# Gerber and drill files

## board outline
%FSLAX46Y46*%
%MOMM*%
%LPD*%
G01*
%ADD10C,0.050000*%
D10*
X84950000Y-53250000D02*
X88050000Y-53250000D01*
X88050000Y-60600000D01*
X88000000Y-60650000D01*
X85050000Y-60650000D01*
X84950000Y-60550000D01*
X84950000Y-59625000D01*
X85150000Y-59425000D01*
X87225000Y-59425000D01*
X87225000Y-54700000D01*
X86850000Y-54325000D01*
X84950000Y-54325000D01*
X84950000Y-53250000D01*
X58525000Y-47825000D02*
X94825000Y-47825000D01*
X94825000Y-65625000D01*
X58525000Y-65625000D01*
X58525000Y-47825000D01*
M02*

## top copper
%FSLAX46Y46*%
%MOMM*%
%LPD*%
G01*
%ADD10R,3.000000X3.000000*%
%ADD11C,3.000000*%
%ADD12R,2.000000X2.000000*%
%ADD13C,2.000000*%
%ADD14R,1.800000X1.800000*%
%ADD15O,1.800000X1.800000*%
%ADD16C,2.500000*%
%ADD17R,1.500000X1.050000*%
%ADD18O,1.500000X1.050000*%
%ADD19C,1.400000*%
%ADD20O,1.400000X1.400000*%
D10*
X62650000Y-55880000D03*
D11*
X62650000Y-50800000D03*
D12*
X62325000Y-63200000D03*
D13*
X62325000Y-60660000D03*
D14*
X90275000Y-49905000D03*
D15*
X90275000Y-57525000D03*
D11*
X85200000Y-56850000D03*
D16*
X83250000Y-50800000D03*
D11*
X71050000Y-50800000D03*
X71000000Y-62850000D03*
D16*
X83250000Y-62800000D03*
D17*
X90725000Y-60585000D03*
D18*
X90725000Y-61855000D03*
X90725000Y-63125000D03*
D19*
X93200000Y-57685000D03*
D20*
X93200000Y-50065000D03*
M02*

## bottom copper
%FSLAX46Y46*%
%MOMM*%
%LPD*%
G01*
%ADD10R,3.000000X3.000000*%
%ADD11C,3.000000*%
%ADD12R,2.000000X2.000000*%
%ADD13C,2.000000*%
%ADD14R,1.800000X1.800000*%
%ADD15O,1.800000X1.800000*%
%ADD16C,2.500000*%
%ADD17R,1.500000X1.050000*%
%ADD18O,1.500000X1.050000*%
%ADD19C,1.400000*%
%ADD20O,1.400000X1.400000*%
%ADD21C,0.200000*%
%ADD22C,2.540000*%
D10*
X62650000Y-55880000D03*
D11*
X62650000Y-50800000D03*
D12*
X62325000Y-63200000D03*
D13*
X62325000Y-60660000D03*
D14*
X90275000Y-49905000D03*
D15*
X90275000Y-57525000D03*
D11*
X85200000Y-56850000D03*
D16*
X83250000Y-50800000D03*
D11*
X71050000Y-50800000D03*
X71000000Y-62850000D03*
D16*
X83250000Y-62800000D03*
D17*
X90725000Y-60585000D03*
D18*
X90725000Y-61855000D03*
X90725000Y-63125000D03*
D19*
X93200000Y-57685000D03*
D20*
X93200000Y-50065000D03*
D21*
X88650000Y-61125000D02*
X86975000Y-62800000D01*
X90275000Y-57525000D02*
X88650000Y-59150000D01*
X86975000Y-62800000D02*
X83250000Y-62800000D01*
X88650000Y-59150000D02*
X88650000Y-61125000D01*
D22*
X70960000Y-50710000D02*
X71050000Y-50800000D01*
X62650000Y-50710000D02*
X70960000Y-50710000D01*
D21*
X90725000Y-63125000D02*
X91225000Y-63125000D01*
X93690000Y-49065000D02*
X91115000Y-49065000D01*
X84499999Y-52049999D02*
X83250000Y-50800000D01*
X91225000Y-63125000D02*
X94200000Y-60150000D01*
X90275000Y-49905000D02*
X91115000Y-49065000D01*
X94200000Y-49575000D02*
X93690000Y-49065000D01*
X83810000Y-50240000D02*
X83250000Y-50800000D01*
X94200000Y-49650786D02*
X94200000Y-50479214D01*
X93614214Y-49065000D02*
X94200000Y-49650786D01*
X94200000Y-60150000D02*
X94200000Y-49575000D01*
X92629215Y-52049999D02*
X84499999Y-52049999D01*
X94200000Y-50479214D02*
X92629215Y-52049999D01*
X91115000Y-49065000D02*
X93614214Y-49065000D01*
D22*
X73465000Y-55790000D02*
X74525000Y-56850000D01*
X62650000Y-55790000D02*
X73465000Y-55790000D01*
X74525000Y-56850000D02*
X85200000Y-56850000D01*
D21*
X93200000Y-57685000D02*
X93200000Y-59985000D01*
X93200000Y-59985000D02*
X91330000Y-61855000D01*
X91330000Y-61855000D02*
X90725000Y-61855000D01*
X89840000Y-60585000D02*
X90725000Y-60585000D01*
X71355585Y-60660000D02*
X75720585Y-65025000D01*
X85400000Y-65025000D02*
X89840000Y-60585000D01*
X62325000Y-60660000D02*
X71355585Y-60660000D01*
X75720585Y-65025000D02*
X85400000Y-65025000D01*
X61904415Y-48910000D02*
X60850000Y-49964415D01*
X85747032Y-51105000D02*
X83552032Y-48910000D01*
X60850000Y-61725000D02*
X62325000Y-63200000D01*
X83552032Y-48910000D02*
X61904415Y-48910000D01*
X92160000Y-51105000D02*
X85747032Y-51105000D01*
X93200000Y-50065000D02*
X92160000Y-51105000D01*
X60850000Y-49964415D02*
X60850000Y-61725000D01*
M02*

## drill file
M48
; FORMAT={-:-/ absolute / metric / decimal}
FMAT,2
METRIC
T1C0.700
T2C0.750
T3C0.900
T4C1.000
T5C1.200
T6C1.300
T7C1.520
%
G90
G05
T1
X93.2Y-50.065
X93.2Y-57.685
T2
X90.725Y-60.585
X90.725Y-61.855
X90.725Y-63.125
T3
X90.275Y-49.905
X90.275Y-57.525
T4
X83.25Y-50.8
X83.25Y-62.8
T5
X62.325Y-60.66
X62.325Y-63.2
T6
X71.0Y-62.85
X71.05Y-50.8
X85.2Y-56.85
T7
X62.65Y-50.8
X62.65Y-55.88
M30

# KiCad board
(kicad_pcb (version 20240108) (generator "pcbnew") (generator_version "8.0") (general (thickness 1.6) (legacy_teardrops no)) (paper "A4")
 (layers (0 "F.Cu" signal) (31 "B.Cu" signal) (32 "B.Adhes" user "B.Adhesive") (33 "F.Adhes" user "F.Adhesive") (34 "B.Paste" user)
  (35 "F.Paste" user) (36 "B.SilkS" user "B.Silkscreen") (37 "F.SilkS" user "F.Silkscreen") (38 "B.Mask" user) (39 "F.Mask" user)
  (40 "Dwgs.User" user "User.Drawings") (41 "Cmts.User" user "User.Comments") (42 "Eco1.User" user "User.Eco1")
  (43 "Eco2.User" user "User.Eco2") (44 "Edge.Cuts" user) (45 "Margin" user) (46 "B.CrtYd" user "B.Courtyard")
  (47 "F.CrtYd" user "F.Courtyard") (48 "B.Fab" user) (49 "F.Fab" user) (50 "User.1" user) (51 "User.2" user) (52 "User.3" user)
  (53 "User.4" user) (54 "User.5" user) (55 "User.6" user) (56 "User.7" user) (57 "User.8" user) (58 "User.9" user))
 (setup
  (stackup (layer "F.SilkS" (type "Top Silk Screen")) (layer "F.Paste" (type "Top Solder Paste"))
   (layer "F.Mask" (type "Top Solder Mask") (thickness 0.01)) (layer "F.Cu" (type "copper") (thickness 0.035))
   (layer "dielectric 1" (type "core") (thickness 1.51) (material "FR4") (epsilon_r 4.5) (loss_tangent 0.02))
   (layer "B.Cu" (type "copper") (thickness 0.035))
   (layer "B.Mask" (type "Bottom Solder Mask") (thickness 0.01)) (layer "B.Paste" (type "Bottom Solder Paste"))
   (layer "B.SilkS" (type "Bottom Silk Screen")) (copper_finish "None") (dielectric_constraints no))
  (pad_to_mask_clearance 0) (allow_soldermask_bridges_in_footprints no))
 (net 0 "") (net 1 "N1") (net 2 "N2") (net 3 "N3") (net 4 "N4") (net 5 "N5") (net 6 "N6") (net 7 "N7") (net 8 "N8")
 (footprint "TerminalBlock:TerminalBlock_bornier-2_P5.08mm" (layer "F.Cu") (at 62.65 55.88 90)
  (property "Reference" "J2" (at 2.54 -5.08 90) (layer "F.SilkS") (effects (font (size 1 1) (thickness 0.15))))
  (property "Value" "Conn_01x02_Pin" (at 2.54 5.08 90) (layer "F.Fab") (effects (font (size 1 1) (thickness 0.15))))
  (pad "1" thru_hole rect (at 0 0 90) (size 3 3) (drill 1.52) (layers "*.Cu" "*.Mask") (remove_unused_layers no) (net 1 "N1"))
  (pad "2" thru_hole circle (at 5.08 0 90) (size 3 3) (drill 1.52) (layers "*.Cu" "*.Mask") (remove_unused_layers no) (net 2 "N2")))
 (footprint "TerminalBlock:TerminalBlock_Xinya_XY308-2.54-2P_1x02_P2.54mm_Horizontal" (layer "F.Cu") (at 62.325 63.2 90)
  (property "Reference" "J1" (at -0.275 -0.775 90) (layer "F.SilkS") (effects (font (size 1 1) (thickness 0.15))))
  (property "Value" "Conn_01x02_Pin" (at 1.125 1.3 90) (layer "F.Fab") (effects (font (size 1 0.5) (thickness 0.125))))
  (pad "1" thru_hole rect (at 0 0 90) (size 2 2) (drill 1.2) (layers "*.Cu" "*.Mask") (remove_unused_layers no) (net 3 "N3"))
  (pad "2" thru_hole circle (at 2.54 0 90) (size 2 2) (drill 1.2) (layers "*.Cu" "*.Mask") (remove_unused_layers no) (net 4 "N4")))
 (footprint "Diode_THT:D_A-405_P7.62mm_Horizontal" (layer "F.Cu") (at 90.275 49.905 -90)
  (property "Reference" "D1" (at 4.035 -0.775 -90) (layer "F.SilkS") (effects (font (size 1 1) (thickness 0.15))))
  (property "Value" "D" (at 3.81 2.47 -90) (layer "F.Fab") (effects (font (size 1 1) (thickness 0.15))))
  (pad "1" thru_hole rect (at 0 0 270) (size 1.8 1.8) (drill 0.9) (layers "*.Cu" "*.Mask") (remove_unused_layers no) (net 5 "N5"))
  (pad "2" thru_hole oval (at 7.62 0 270) (size 1.8 1.8) (drill 0.9) (layers "*.Cu" "*.Mask") (remove_unused_layers no) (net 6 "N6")))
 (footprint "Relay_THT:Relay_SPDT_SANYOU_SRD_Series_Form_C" (layer "F.Cu") (at 85.2 56.85 180)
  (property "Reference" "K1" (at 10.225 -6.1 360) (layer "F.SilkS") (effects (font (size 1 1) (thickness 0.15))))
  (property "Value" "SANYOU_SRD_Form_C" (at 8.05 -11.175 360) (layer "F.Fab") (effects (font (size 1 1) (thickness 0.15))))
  (pad "1" thru_hole circle (at 0 0 270) (size 3 3) (drill 1.3) (layers "*.Cu" "*.Mask") (remove_unused_layers no) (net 1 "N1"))
  (pad "2" thru_hole circle (at 1.95 6.05 270) (size 2.5 2.5) (drill 1) (layers "*.Cu" "*.Mask") (remove_unused_layers no) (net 5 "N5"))
  (pad "3" thru_hole circle (at 14.15 6.05 270) (size 3 3) (drill 1.3) (layers "*.Cu" "*.Mask") (remove_unused_layers no) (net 2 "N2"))
  (pad "4" thru_hole circle (at 14.2 -6 270) (size 3 3) (drill 1.3) (layers "*.Cu" "*.Mask") (remove_unused_layers no) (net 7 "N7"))
  (pad "5" thru_hole circle (at 1.95 -5.95 270) (size 2.5 2.5) (drill 1) (layers "*.Cu" "*.Mask") (remove_unused_layers no) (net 6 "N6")))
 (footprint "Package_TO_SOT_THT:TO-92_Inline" (layer "F.Cu") (at 90.725 60.585 -90)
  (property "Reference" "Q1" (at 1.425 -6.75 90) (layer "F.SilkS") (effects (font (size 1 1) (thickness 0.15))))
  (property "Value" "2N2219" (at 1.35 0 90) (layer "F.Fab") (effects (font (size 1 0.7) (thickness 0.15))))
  (pad "1" thru_hole rect (at 0 0 270) (size 1.05 1.5) (drill 0.75) (layers "*.Cu" "*.Mask") (remove_unused_layers no) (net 4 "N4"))
  (pad "2" thru_hole oval (at 1.27 0 270) (size 1.05 1.5) (drill 0.75) (layers "*.Cu" "*.Mask") (remove_unused_layers no) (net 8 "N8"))
  (pad "3" thru_hole oval (at 2.54 0 270) (size 1.05 1.5) (drill 0.75) (layers "*.Cu" "*.Mask") (remove_unused_layers no) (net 5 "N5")))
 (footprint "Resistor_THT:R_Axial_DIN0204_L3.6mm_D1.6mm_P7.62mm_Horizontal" (layer "F.Cu") (at 93.2 57.685 90)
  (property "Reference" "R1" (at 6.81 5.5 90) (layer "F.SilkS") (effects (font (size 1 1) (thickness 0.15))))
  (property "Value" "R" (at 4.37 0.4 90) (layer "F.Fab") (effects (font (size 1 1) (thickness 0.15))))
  (pad "1" thru_hole circle (at 0 0 90) (size 1.4 1.4) (drill 0.7) (layers "*.Cu" "*.Mask") (remove_unused_layers no) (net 8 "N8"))
  (pad "2" thru_hole oval (at 7.62 0 90) (size 1.4 1.4) (drill 0.7) (layers "*.Cu" "*.Mask") (remove_unused_layers no) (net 3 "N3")))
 (gr_poly
  (pts (xy 84.95 53.25) (xy 88.05 53.25) (xy 88.05 60.6) (xy 88 60.65) (xy 85.05 60.65) (xy 84.95 60.55) (xy 84.95 59.625) (xy 85.15 59.425)
   (xy 87.225 59.425) (xy 87.225 54.7) (xy 86.85 54.325) (xy 84.95 54.325))
  (stroke (width 0.05) (type solid)) (fill none) (layer "Edge.Cuts"))
 (gr_rect (start 58.525 47.825) (end 94.825 65.625) (stroke (width 0.05) (type default)) (fill none) (layer "Edge.Cuts"))
 (segment (start 88.65 61.125) (end 86.975 62.8) (width 0.2) (layer "B.Cu") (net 6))
 (segment (start 90.275 57.525) (end 88.65 59.15) (width 0.2) (layer "B.Cu") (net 6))
 (segment (start 86.975 62.8) (end 83.25 62.8) (width 0.2) (layer "B.Cu") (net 6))
 (segment (start 88.65 59.15) (end 88.65 61.125) (width 0.2) (layer "B.Cu") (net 6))
 (segment (start 70.96 50.71) (end 71.05 50.8) (width 2.54) (layer "B.Cu") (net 2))
 (segment (start 62.65 50.71) (end 70.96 50.71) (width 2.54) (layer "B.Cu") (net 2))
 (segment (start 90.725 63.125) (end 91.225 63.125) (width 0.2) (layer "B.Cu") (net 5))
 (segment (start 93.69 49.065) (end 91.115 49.065) (width 0.2) (layer "B.Cu") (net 5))
 (segment (start 84.499999 52.049999) (end 83.25 50.8) (width 0.2) (layer "B.Cu") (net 5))
 (segment (start 91.225 63.125) (end 94.2 60.15) (width 0.2) (layer "B.Cu") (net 5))
 (segment (start 90.275 49.905) (end 91.115 49.065) (width 0.2) (layer "B.Cu") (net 5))
 (segment (start 94.2 49.575) (end 93.69 49.065) (width 0.2) (layer "B.Cu") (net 5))
 (segment (start 83.81 50.24) (end 83.25 50.8) (width 0.2) (layer "B.Cu") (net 5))
 (segment (start 94.2 49.650786) (end 94.2 50.479214) (width 0.2) (layer "B.Cu") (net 5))
 (segment (start 93.614214 49.065) (end 94.2 49.650786) (width 0.2) (layer "B.Cu") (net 5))
 (segment (start 94.2 60.15) (end 94.2 49.575) (width 0.2) (layer "B.Cu") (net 5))
 (segment (start 92.629215 52.049999) (end 84.499999 52.049999) (width 0.2) (layer "B.Cu") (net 5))
 (segment (start 94.2 50.479214) (end 92.629215 52.049999) (width 0.2) (layer "B.Cu") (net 5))
 (segment (start 91.115 49.065) (end 93.614214 49.065) (width 0.2) (layer "B.Cu") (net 5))
 (segment (start 73.465 55.79) (end 74.525 56.85) (width 2.54) (layer "B.Cu") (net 1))
 (segment (start 62.65 55.79) (end 73.465 55.79) (width 2.54) (layer "B.Cu") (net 1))
 (segment (start 74.525 56.85) (end 85.2 56.85) (width 2.54) (layer "B.Cu") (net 1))
 (segment (start 93.2 57.685) (end 93.2 59.985) (width 0.2) (layer "B.Cu") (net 8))
 (segment (start 93.2 59.985) (end 91.33 61.855) (width 0.2) (layer "B.Cu") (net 8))
 (segment (start 91.33 61.855) (end 90.725 61.855) (width 0.2) (layer "B.Cu") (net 8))
 (segment (start 89.84 60.585) (end 90.725 60.585) (width 0.2) (layer "B.Cu") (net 4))
 (segment (start 71.355585 60.66) (end 75.720585 65.025) (width 0.2) (layer "B.Cu") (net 4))
 (segment (start 85.4 65.025) (end 89.84 60.585) (width 0.2) (layer "B.Cu") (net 4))
 (segment (start 62.325 60.66) (end 71.355585 60.66) (width 0.2) (layer "B.Cu") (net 4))
 (segment (start 75.720585 65.025) (end 85.4 65.025) (width 0.2) (layer "B.Cu") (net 4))
 (segment (start 61.904415 48.91) (end 60.85 49.964415) (width 0.2) (layer "B.Cu") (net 3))
 (segment (start 85.747032 51.105) (end 83.552032 48.91) (width 0.2) (layer "B.Cu") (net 3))
 (segment (start 60.85 61.725) (end 62.325 63.2) (width 0.2) (layer "B.Cu") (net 3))
 (segment (start 83.552032 48.91) (end 61.904415 48.91) (width 0.2) (layer "B.Cu") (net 3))
 (segment (start 92.16 51.105) (end 85.747032 51.105) (width 0.2) (layer "B.Cu") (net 3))
 (segment (start 93.2 50.065) (end 92.16 51.105) (width 0.2) (layer "B.Cu") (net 3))
 (segment (start 60.85 49.964415) (end 60.85 61.725) (width 0.2) (layer "B.Cu") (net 3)))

